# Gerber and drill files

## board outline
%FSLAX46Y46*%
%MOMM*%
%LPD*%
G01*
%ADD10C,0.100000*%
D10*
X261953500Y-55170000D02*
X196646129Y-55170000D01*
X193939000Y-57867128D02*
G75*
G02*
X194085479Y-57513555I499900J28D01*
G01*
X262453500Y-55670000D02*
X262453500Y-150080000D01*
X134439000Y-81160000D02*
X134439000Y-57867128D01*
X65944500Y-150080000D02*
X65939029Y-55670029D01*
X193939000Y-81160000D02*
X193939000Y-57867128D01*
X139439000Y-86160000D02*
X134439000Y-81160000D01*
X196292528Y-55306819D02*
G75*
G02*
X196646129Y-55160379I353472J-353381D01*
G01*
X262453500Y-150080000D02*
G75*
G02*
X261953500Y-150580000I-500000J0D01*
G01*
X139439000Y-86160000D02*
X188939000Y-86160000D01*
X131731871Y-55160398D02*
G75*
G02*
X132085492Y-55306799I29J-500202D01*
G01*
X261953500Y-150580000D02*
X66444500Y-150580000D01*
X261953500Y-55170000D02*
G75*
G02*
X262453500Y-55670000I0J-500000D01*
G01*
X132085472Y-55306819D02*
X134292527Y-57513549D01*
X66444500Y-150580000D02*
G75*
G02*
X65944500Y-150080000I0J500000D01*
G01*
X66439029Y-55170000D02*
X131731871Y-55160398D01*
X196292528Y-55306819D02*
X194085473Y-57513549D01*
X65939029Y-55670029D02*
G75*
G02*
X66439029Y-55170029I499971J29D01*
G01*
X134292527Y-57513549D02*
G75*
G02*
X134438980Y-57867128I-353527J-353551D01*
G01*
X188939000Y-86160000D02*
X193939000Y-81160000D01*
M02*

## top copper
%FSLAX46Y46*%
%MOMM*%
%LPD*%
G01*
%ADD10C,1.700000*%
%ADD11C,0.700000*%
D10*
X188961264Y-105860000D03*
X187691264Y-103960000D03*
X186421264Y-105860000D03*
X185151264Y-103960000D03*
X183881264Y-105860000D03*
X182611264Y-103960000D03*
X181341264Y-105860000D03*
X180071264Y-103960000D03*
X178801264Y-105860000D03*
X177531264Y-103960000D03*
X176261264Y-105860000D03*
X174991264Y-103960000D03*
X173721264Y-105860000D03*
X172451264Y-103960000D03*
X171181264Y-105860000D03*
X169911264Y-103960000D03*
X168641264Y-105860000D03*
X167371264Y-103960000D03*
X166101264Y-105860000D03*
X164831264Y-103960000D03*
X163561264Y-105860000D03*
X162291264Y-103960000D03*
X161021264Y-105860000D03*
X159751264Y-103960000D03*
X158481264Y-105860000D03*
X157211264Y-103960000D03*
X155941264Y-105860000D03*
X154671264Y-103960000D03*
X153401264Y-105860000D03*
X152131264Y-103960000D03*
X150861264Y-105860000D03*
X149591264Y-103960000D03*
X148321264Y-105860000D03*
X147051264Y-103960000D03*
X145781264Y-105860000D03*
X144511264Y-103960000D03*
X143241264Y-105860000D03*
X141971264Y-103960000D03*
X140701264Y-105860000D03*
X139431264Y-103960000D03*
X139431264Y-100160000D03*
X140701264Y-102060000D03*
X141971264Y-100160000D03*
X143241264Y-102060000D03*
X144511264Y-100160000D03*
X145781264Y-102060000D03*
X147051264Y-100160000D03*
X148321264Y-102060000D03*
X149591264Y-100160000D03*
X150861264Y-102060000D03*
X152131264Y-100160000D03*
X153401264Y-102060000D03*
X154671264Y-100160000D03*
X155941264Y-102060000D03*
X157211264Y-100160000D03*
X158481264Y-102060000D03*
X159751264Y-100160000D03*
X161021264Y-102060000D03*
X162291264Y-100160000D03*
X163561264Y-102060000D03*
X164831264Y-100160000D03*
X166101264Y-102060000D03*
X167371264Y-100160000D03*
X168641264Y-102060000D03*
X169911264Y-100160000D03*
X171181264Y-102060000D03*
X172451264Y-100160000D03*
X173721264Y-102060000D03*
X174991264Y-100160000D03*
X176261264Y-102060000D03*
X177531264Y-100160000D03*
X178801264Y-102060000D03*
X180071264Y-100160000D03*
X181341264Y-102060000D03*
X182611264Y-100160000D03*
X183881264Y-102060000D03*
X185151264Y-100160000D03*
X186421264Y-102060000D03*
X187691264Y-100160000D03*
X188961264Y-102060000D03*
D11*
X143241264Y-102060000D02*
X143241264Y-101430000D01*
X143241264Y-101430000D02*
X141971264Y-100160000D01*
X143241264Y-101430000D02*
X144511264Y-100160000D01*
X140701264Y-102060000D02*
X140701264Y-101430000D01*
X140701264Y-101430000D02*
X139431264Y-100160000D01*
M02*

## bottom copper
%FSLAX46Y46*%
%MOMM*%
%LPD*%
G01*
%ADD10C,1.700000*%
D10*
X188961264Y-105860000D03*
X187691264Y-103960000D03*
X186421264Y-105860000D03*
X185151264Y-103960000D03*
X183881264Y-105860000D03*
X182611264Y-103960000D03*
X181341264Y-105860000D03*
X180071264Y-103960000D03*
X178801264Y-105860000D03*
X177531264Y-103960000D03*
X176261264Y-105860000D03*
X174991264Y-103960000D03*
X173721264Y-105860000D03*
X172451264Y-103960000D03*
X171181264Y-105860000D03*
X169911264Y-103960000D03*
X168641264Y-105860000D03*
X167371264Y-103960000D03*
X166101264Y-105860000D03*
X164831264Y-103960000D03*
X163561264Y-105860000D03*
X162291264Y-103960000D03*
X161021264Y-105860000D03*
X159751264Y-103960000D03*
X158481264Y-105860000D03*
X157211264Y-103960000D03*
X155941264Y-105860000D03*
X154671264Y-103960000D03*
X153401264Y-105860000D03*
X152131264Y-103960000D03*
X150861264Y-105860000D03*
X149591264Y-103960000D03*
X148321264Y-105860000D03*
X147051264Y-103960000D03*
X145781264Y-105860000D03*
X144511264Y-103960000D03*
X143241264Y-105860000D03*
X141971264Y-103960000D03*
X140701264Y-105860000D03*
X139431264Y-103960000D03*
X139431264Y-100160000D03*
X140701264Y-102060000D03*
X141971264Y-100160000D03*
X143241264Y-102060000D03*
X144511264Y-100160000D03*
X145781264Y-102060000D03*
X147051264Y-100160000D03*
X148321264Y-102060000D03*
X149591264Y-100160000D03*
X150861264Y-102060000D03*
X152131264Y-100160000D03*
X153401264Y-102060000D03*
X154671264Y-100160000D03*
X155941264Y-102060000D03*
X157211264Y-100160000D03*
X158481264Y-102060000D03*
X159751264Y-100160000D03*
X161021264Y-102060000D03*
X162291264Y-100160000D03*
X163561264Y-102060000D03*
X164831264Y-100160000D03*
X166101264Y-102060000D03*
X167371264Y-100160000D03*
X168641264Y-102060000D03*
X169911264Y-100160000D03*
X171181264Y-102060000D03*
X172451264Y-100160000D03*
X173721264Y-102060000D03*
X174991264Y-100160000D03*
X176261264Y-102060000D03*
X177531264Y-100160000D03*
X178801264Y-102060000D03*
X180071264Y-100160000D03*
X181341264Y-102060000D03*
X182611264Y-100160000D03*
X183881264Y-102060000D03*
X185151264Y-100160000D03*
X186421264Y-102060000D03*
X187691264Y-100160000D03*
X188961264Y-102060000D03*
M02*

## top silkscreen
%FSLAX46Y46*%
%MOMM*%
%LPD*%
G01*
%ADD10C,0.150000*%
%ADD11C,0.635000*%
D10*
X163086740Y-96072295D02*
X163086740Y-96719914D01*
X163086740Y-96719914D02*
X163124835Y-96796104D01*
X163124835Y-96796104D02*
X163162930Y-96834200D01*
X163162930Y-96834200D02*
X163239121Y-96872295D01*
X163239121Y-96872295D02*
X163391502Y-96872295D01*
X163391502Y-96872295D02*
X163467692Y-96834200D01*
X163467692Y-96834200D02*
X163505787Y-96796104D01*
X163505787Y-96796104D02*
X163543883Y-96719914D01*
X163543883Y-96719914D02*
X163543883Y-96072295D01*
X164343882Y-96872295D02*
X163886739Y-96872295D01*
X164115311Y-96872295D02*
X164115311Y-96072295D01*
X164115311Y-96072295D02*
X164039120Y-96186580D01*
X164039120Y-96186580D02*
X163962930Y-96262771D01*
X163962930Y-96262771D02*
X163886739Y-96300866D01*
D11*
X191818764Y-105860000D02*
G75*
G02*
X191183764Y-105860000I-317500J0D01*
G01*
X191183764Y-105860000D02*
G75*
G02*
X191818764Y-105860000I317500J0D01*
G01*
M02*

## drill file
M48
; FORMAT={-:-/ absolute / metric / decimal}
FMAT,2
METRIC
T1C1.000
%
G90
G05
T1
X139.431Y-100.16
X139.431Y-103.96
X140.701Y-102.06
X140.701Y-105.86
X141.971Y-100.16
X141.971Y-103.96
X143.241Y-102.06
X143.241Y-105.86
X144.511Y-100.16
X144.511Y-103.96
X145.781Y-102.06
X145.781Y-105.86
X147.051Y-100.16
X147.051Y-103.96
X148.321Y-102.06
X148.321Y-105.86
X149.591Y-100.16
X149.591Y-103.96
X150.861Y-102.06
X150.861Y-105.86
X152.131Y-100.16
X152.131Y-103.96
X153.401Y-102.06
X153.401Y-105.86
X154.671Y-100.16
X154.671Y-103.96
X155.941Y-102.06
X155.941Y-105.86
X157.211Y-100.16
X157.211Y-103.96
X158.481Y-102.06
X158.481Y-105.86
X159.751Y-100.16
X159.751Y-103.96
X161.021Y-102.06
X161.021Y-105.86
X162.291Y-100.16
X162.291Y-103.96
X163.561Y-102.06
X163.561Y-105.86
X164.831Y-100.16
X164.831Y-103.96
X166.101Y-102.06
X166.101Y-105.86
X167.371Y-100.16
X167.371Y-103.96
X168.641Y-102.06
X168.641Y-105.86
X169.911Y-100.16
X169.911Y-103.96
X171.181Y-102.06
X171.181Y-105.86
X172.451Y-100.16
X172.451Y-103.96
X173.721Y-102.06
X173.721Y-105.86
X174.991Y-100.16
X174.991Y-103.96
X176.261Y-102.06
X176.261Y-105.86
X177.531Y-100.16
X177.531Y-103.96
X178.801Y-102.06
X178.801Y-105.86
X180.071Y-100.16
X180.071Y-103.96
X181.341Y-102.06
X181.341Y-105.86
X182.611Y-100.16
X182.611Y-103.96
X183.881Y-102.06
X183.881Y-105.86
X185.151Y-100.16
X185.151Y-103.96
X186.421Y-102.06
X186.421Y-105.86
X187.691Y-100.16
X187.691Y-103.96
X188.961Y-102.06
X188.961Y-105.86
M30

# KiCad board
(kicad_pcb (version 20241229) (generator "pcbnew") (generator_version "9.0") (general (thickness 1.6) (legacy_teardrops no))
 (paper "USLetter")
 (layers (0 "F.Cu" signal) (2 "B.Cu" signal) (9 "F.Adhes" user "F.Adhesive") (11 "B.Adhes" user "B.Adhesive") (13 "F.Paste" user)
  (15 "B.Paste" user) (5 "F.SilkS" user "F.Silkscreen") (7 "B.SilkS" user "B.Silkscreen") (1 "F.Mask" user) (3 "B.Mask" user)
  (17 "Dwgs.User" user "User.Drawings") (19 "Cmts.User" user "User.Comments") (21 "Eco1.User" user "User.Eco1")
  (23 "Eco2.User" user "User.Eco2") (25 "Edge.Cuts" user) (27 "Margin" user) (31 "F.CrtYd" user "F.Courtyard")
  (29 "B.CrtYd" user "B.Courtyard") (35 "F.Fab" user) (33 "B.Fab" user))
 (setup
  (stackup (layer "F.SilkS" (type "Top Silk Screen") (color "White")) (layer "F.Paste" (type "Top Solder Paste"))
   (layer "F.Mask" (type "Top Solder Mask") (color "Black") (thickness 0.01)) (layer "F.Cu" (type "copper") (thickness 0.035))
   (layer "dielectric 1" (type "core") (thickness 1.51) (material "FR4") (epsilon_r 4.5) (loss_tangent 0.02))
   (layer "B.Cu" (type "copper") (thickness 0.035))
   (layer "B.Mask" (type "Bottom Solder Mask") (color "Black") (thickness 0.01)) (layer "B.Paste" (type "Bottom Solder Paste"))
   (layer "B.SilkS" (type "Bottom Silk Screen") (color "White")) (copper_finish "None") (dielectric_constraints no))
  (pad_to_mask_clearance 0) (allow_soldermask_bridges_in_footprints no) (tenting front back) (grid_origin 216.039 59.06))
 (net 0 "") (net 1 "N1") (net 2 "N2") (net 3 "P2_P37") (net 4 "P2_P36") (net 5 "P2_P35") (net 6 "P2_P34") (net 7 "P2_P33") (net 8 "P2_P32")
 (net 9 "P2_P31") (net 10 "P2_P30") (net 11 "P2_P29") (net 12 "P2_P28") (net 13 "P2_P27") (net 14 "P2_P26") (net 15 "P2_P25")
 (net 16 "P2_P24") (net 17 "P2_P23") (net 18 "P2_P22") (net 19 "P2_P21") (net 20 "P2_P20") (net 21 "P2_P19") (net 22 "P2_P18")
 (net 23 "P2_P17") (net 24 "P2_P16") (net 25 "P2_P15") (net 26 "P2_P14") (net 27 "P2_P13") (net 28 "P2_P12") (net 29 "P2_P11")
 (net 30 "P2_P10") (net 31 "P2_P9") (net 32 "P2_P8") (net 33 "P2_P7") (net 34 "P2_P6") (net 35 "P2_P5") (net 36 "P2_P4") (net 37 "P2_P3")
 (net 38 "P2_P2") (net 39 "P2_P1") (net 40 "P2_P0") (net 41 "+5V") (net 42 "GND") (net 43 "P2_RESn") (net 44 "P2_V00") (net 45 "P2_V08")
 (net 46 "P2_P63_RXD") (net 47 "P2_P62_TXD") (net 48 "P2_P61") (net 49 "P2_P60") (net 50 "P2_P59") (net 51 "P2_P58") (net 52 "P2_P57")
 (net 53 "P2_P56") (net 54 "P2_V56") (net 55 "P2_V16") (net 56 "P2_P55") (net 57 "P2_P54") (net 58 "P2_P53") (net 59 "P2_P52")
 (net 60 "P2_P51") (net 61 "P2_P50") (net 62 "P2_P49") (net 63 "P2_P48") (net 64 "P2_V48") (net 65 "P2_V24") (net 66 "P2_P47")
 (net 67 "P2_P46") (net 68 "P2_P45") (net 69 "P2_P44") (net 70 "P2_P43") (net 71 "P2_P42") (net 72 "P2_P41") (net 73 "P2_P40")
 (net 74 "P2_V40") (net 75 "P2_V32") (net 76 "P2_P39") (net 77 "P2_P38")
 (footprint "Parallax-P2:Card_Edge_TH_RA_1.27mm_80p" (layer "F.Cu") (at 164.196264 103.01)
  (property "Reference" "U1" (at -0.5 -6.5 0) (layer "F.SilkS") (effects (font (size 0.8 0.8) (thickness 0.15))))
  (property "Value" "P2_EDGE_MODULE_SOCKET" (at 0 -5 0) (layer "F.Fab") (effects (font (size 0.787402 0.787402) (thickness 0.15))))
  (fp_circle (center 27.305 2.85) (end 27.94 2.85) (stroke (width 0) (type solid)) (fill yes) (layer "F.SilkS"))
  (pad "1" thru_hole circle (at 24.765 2.85) (size 1.7 1.7) (drill 1) (layers "*.Cu" "*.Mask") (remove_unused_layers no) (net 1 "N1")
   (solder_mask_margin 0.102))
  (pad "2" thru_hole circle (at 23.495 0.95) (size 1.7 1.7) (drill 1) (layers "*.Cu" "*.Mask") (remove_unused_layers no) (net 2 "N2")
   (solder_mask_margin 0.102))
  (pad "3" thru_hole circle (at 22.225 2.85) (size 1.7 1.7) (drill 1) (layers "*.Cu" "*.Mask") (remove_unused_layers no) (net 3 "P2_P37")
   (solder_mask_margin 0.102))
  (pad "4" thru_hole circle (at 20.955 0.95) (size 1.7 1.7) (drill 1) (layers "*.Cu" "*.Mask") (remove_unused_layers no) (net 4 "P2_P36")
   (solder_mask_margin 0.102))
  (pad "5" thru_hole circle (at 19.685 2.85) (size 1.7 1.7) (drill 1) (layers "*.Cu" "*.Mask") (remove_unused_layers no) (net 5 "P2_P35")
   (solder_mask_margin 0.102))
  (pad "6" thru_hole circle (at 18.415 0.95) (size 1.7 1.7) (drill 1) (layers "*.Cu" "*.Mask") (remove_unused_layers no) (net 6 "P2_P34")
   (solder_mask_margin 0.102))
  (pad "7" thru_hole circle (at 17.145 2.85) (size 1.7 1.7) (drill 1) (layers "*.Cu" "*.Mask") (remove_unused_layers no) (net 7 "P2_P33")
   (solder_mask_margin 0.102))
  (pad "8" thru_hole circle (at 15.875 0.95) (size 1.7 1.7) (drill 1) (layers "*.Cu" "*.Mask") (remove_unused_layers no) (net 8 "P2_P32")
   (solder_mask_margin 0.102))
  (pad "9" thru_hole circle (at 14.605 2.85) (size 1.7 1.7) (drill 1) (layers "*.Cu" "*.Mask") (remove_unused_layers no) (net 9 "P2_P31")
   (solder_mask_margin 0.102))
  (pad "10" thru_hole circle (at 13.335 0.95) (size 1.7 1.7) (drill 1) (layers "*.Cu" "*.Mask") (remove_unused_layers no) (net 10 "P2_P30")
   (solder_mask_margin 0.102))
  (pad "11" thru_hole circle (at 12.065 2.85) (size 1.7 1.7) (drill 1) (layers "*.Cu" "*.Mask") (remove_unused_layers no) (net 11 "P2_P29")
   (solder_mask_margin 0.102))
  (pad "12" thru_hole circle (at 10.795 0.95) (size 1.7 1.7) (drill 1) (layers "*.Cu" "*.Mask") (remove_unused_layers no) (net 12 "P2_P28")
   (solder_mask_margin 0.102))
  (pad "13" thru_hole circle (at 9.525 2.85) (size 1.7 1.7) (drill 1) (layers "*.Cu" "*.Mask") (remove_unused_layers no) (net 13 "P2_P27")
   (solder_mask_margin 0.102))
  (pad "14" thru_hole circle (at 8.255 0.95) (size 1.7 1.7) (drill 1) (layers "*.Cu" "*.Mask") (remove_unused_layers no) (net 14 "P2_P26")
   (solder_mask_margin 0.102))
  (pad "15" thru_hole circle (at 6.985 2.85) (size 1.7 1.7) (drill 1) (layers "*.Cu" "*.Mask") (remove_unused_layers no) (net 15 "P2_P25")
   (solder_mask_margin 0.102))
  (pad "16" thru_hole circle (at 5.715 0.95) (size 1.7 1.7) (drill 1) (layers "*.Cu" "*.Mask") (remove_unused_layers no) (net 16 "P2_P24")
   (solder_mask_margin 0.102))
  (pad "17" thru_hole circle (at 4.445 2.85) (size 1.7 1.7) (drill 1) (layers "*.Cu" "*.Mask") (remove_unused_layers no) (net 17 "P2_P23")
   (solder_mask_margin 0.102))
  (pad "18" thru_hole circle (at 3.175 0.95) (size 1.7 1.7) (drill 1) (layers "*.Cu" "*.Mask") (remove_unused_layers no) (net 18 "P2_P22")
   (solder_mask_margin 0.102))
  (pad "19" thru_hole circle (at 1.905 2.85) (size 1.7 1.7) (drill 1) (layers "*.Cu" "*.Mask") (remove_unused_layers no) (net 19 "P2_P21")
   (solder_mask_margin 0.102))
  (pad "20" thru_hole circle (at 0.635 0.95) (size 1.7 1.7) (drill 1) (layers "*.Cu" "*.Mask") (remove_unused_layers no) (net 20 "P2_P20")
   (solder_mask_margin 0.102))
  (pad "21" thru_hole circle (at -0.635 2.85) (size 1.7 1.7) (drill 1) (layers "*.Cu" "*.Mask") (remove_unused_layers no) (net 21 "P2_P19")
   (solder_mask_margin 0.102))
  (pad "22" thru_hole circle (at -1.905 0.95) (size 1.7 1.7) (drill 1) (layers "*.Cu" "*.Mask") (remove_unused_layers no) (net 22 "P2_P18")
   (solder_mask_margin 0.102))
  (pad "23" thru_hole circle (at -3.175 2.85) (size 1.7 1.7) (drill 1) (layers "*.Cu" "*.Mask") (remove_unused_layers no) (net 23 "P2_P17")
   (solder_mask_margin 0.102))
  (pad "24" thru_hole circle (at -4.445 0.95) (size 1.7 1.7) (drill 1) (layers "*.Cu" "*.Mask") (remove_unused_layers no) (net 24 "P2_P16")
   (solder_mask_margin 0.102))
  (pad "25" thru_hole circle (at -5.715 2.85) (size 1.7 1.7) (drill 1) (layers "*.Cu" "*.Mask") (remove_unused_layers no) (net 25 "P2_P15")
   (solder_mask_margin 0.102))
  (pad "26" thru_hole circle (at -6.985 0.95) (size 1.7 1.7) (drill 1) (layers "*.Cu" "*.Mask") (remove_unused_layers no) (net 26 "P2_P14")
   (solder_mask_margin 0.102))
  (pad "27" thru_hole circle (at -8.255 2.85) (size 1.7 1.7) (drill 1) (layers "*.Cu" "*.Mask") (remove_unused_layers no) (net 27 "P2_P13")
   (solder_mask_margin 0.102))
  (pad "28" thru_hole circle (at -9.525 0.95) (size 1.7 1.7) (drill 1) (layers "*.Cu" "*.Mask") (remove_unused_layers no) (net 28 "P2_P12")
   (solder_mask_margin 0.102))
  (pad "29" thru_hole circle (at -10.795 2.85) (size 1.7 1.7) (drill 1) (layers "*.Cu" "*.Mask") (remove_unused_layers no) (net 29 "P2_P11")
   (solder_mask_margin 0.102))
  (pad "30" thru_hole circle (at -12.065 0.95) (size 1.7 1.7) (drill 1) (layers "*.Cu" "*.Mask") (remove_unused_layers no) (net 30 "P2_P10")
   (solder_mask_margin 0.102))
  (pad "31" thru_hole circle (at -13.335 2.85) (size 1.7 1.7) (drill 1) (layers "*.Cu" "*.Mask") (remove_unused_layers no) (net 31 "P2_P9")
   (solder_mask_margin 0.102))
  (pad "32" thru_hole circle (at -14.605 0.95) (size 1.7 1.7) (drill 1) (layers "*.Cu" "*.Mask") (remove_unused_layers no) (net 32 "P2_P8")
   (solder_mask_margin 0.102))
  (pad "33" thru_hole circle (at -15.875 2.85) (size 1.7 1.7) (drill 1) (layers "*.Cu" "*.Mask") (remove_unused_layers no) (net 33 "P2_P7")
   (solder_mask_margin 0.102))
  (pad "34" thru_hole circle (at -17.145 0.95) (size 1.7 1.7) (drill 1) (layers "*.Cu" "*.Mask") (remove_unused_layers no) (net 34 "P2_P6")
   (solder_mask_margin 0.102))
  (pad "35" thru_hole circle (at -18.415 2.85) (size 1.7 1.7) (drill 1) (layers "*.Cu" "*.Mask") (remove_unused_layers no) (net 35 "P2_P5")
   (solder_mask_margin 0.102))
  (pad "36" thru_hole circle (at -19.685 0.95) (size 1.7 1.7) (drill 1) (layers "*.Cu" "*.Mask") (remove_unused_layers no) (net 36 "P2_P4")
   (solder_mask_margin 0.102))
  (pad "37" thru_hole circle (at -20.955 2.85) (size 1.7 1.7) (drill 1) (layers "*.Cu" "*.Mask") (remove_unused_layers no) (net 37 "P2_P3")
   (solder_mask_margin 0.102))
  (pad "38" thru_hole circle (at -22.225 0.95) (size 1.7 1.7) (drill 1) (layers "*.Cu" "*.Mask") (remove_unused_layers no) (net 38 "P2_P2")
   (solder_mask_margin 0.102))
  (pad "39" thru_hole circle (at -23.495 2.85) (size 1.7 1.7) (drill 1) (layers "*.Cu" "*.Mask") (remove_unused_layers no) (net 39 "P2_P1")
   (solder_mask_margin 0.102))
  (pad "40" thru_hole circle (at -24.765 0.95) (size 1.7 1.7) (drill 1) (layers "*.Cu" "*.Mask") (remove_unused_layers no) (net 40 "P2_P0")
   (solder_mask_margin 0.102))
  (pad "41" thru_hole circle (at -24.765 -2.85) (size 1.7 1.7) (drill 1) (layers "*.Cu" "*.Mask") (remove_unused_layers no) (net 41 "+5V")
   (solder_mask_margin 0.102))
  (pad "42" thru_hole circle (at -23.495 -0.95) (size 1.7 1.7) (drill 1) (layers "*.Cu" "*.Mask") (remove_unused_layers no) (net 41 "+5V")
   (solder_mask_margin 0.102))
  (pad "43" thru_hole circle (at -22.225 -2.85) (size 1.7 1.7) (drill 1) (layers "*.Cu" "*.Mask") (remove_unused_layers no) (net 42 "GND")
   (solder_mask_margin 0.102))
  (pad "44" thru_hole circle (at -20.955 -0.95) (size 1.7 1.7) (drill 1) (layers "*.Cu" "*.Mask") (remove_unused_layers no) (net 42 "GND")
   (solder_mask_margin 0.102))
  (pad "45" thru_hole circle (at -19.685 -2.85) (size 1.7 1.7) (drill 1) (layers "*.Cu" "*.Mask") (remove_unused_layers no) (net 42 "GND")
   (solder_mask_margin 0.102))
  (pad "46" thru_hole circle (at -18.415 -0.95) (size 1.7 1.7) (drill 1) (layers "*.Cu" "*.Mask") (remove_unused_layers no)
   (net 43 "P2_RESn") (solder_mask_margin 0.102))
  (pad "47" thru_hole circle (at -17.145 -2.85) (size 1.7 1.7) (drill 1) (layers "*.Cu" "*.Mask") (remove_unused_layers no)
   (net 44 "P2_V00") (solder_mask_margin 0.102))
  (pad "48" thru_hole circle (at -15.875 -0.95) (size 1.7 1.7) (drill 1) (layers "*.Cu" "*.Mask") (remove_unused_layers no)
   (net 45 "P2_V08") (solder_mask_margin 0.102))
  (pad "49" thru_hole circle (at -14.605 -2.85) (size 1.7 1.7) (drill 1) (layers "*.Cu" "*.Mask") (remove_unused_layers no)
   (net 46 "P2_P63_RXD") (solder_mask_margin 0.102))
  (pad "50" thru_hole circle (at -13.335 -0.95) (size 1.7 1.7) (drill 1) (layers "*.Cu" "*.Mask") (remove_unused_layers no)
   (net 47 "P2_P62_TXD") (solder_mask_margin 0.102))
  (pad "51" thru_hole circle (at -12.065 -2.85) (size 1.7 1.7) (drill 1) (layers "*.Cu" "*.Mask") (remove_unused_layers no)
   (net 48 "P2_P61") (solder_mask_margin 0.102))
  (pad "52" thru_hole circle (at -10.795 -0.95) (size 1.7 1.7) (drill 1) (layers "*.Cu" "*.Mask") (remove_unused_layers no)
   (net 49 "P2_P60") (solder_mask_margin 0.102))
  (pad "53" thru_hole circle (at -9.525 -2.85) (size 1.7 1.7) (drill 1) (layers "*.Cu" "*.Mask") (remove_unused_layers no) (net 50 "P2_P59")
   (solder_mask_margin 0.102))
  (pad "54" thru_hole circle (at -8.255 -0.95) (size 1.7 1.7) (drill 1) (layers "*.Cu" "*.Mask") (remove_unused_layers no) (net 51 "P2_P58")
   (solder_mask_margin 0.102))
  (pad "55" thru_hole circle (at -6.985 -2.85) (size 1.7 1.7) (drill 1) (layers "*.Cu" "*.Mask") (remove_unused_layers no) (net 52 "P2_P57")
   (solder_mask_margin 0.102))
  (pad "56" thru_hole circle (at -5.715 -0.95) (size 1.7 1.7) (drill 1) (layers "*.Cu" "*.Mask") (remove_unused_layers no) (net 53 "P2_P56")
   (solder_mask_margin 0.102))
  (pad "57" thru_hole circle (at -4.445 -2.85) (size 1.7 1.7) (drill 1) (layers "*.Cu" "*.Mask") (remove_unused_layers no) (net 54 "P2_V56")
   (solder_mask_margin 0.102))
  (pad "58" thru_hole circle (at -3.175 -0.95) (size 1.7 1.7) (drill 1) (layers "*.Cu" "*.Mask") (remove_unused_layers no) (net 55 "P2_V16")
   (solder_mask_margin 0.102))
  (pad "59" thru_hole circle (at -1.905 -2.85) (size 1.7 1.7) (drill 1) (layers "*.Cu" "*.Mask") (remove_unused_layers no) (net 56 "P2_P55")
   (solder_mask_margin 0.102))
  (pad "60" thru_hole circle (at -0.635 -0.95) (size 1.7 1.7) (drill 1) (layers "*.Cu" "*.Mask") (remove_unused_layers no) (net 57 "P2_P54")
   (solder_mask_margin 0.102))
  (pad "61" thru_hole circle (at 0.635 -2.85) (size 1.7 1.7) (drill 1) (layers "*.Cu" "*.Mask") (remove_unused_layers no) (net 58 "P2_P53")
   (solder_mask_margin 0.102))
  (pad "62" thru_hole circle (at 1.905 -0.95) (size 1.7 1.7) (drill 1) (layers "*.Cu" "*.Mask") (remove_unused_layers no) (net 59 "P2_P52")
   (solder_mask_margin 0.102))
  (pad "63" thru_hole circle (at 3.175 -2.85) (size 1.7 1.7) (drill 1) (layers "*.Cu" "*.Mask") (remove_unused_layers no) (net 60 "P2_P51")
   (solder_mask_margin 0.102))
  (pad "64" thru_hole circle (at 4.445 -0.95) (size 1.7 1.7) (drill 1) (layers "*.Cu" "*.Mask") (remove_unused_layers no) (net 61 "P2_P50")
   (solder_mask_margin 0.102))
  (pad "65" thru_hole circle (at 5.715 -2.85) (size 1.7 1.7) (drill 1) (layers "*.Cu" "*.Mask") (remove_unused_layers no) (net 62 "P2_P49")
   (solder_mask_margin 0.102))
  (pad "66" thru_hole circle (at 6.985 -0.95) (size 1.7 1.7) (drill 1) (layers "*.Cu" "*.Mask") (remove_unused_layers no) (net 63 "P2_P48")
   (solder_mask_margin 0.102))
  (pad "67" thru_hole circle (at 8.255 -2.85) (size 1.7 1.7) (drill 1) (layers "*.Cu" "*.Mask") (remove_unused_layers no) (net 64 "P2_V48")
   (solder_mask_margin 0.102))
  (pad "68" thru_hole circle (at 9.525 -0.95) (size 1.7 1.7) (drill 1) (layers "*.Cu" "*.Mask") (remove_unused_layers no) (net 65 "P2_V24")
   (solder_mask_margin 0.102))
  (pad "69" thru_hole circle (at 10.795 -2.85) (size 1.7 1.7) (drill 1) (layers "*.Cu" "*.Mask") (remove_unused_layers no) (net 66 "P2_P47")
   (solder_mask_margin 0.102))
  (pad "70" thru_hole circle (at 12.065 -0.95) (size 1.7 1.7) (drill 1) (layers "*.Cu" "*.Mask") (remove_unused_layers no) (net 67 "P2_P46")
   (solder_mask_margin 0.102))
  (pad "71" thru_hole circle (at 13.335 -2.85) (size 1.7 1.7) (drill 1) (layers "*.Cu" "*.Mask") (remove_unused_layers no) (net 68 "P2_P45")
   (solder_mask_margin 0.102))
  (pad "72" thru_hole circle (at 14.605 -0.95) (size 1.7 1.7) (drill 1) (layers "*.Cu" "*.Mask") (remove_unused_layers no) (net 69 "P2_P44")
   (solder_mask_margin 0.102))
  (pad "73" thru_hole circle (at 15.875 -2.85) (size 1.7 1.7) (drill 1) (layers "*.Cu" "*.Mask") (remove_unused_layers no) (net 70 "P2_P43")
   (solder_mask_margin 0.102))
  (pad "74" thru_hole circle (at 17.145 -0.95) (size 1.7 1.7) (drill 1) (layers "*.Cu" "*.Mask") (remove_unused_layers no) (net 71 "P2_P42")
   (solder_mask_margin 0.102))
  (pad "75" thru_hole circle (at 18.415 -2.85) (size 1.7 1.7) (drill 1) (layers "*.Cu" "*.Mask") (remove_unused_layers no) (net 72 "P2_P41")
   (solder_mask_margin 0.102))
  (pad "76" thru_hole circle (at 19.685 -0.95) (size 1.7 1.7) (drill 1) (layers "*.Cu" "*.Mask") (remove_unused_layers no) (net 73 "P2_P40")
   (solder_mask_margin 0.102))
  (pad "77" thru_hole circle (at 20.955 -2.85) (size 1.7 1.7) (drill 1) (layers "*.Cu" "*.Mask") (remove_unused_layers no) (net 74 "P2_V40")
   (solder_mask_margin 0.102))
  (pad "78" thru_hole circle (at 22.225 -0.95) (size 1.7 1.7) (drill 1) (layers "*.Cu" "*.Mask") (remove_unused_layers no) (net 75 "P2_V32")
   (solder_mask_margin 0.102))
  (pad "79" thru_hole circle (at 23.495 -2.85) (size 1.7 1.7) (drill 1) (layers "*.Cu" "*.Mask") (remove_unused_layers no) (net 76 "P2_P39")
   (solder_mask_margin 0.102))
  (pad "80" thru_hole circle (at 24.765 -0.95) (size 1.7 1.7) (drill 1) (layers "*.Cu" "*.Mask") (remove_unused_layers no) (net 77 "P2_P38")
   (solder_mask_margin 0.102)))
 (gr_line (start 261.9535 55.17) (end 196.646129 55.17) (stroke (width 0.1) (type solid)) (layer "Edge.Cuts"))
 (gr_arc (start 193.939 57.867128) (mid 193.977058 57.675763) (end 194.085473 57.513549) (stroke (width 0.1) (type default))
  (layer "Edge.Cuts"))
 (gr_line (start 262.4535 55.67) (end 262.4535 150.08) (stroke (width 0.1) (type solid)) (layer "Edge.Cuts"))
 (gr_line (start 134.439 81.16) (end 134.439 57.867128) (stroke (width 0.1) (type solid)) (layer "Edge.Cuts"))
 (gr_line (start 65.9445 150.08) (end 65.939029 55.670029) (stroke (width 0.1) (type solid)) (layer "Edge.Cuts"))
 (gr_line (start 193.939 81.16) (end 193.939 57.867128) (stroke (width 0.1) (type solid)) (layer "Edge.Cuts"))
 (gr_line (start 139.439 86.16) (end 134.439 81.16) (stroke (width 0.1) (type default)) (layer "Edge.Cuts"))
 (gr_arc (start 196.292528 55.306819) (mid 196.454762 55.198423) (end 196.646129 55.160398) (stroke (width 0.1) (type default))
  (layer "Edge.Cuts"))
 (gr_arc (start 262.4535 150.08) (mid 262.307053 150.433553) (end 261.9535 150.58) (stroke (width 0.1) (type solid)) (layer "Edge.Cuts"))
 (gr_line (start 139.439 86.16) (end 188.939 86.16) (stroke (width 0.1) (type default)) (layer "Edge.Cuts"))
 (gr_arc (start 131.731871 55.160398) (mid 131.923226 55.198452) (end 132.085472 55.306819) (stroke (width 0.1) (type default))
  (layer "Edge.Cuts"))
 (gr_line (start 261.9535 150.58) (end 66.4445 150.58) (stroke (width 0.1) (type solid)) (layer "Edge.Cuts"))
 (gr_arc (start 261.9535 55.17) (mid 262.307053 55.316447) (end 262.4535 55.67) (stroke (width 0.1) (type solid)) (layer "Edge.Cuts"))
 (gr_line (start 132.085472 55.306819) (end 134.292527 57.513549) (stroke (width 0.1) (type default)) (layer "Edge.Cuts"))
 (gr_arc (start 66.4445 150.58) (mid 66.090947 150.433553) (end 65.9445 150.08) (stroke (width 0.1) (type solid)) (layer "Edge.Cuts"))
 (gr_line (start 66.439029 55.17) (end 131.731871 55.160398) (stroke (width 0.1) (type default)) (layer "Edge.Cuts"))
 (gr_line (start 196.292528 55.306819) (end 194.085473 57.513549) (stroke (width 0.1) (type default)) (layer "Edge.Cuts"))
 (gr_arc (start 65.939029 55.670029) (mid 66.085467 55.316467) (end 66.439029 55.17) (stroke (width 0.1) (type solid)) (layer "Edge.Cuts"))
 (gr_arc (start 134.292527 57.513549) (mid 134.400932 57.67577) (end 134.439 57.867128) (stroke (width 0.1) (type default))
  (layer "Edge.Cuts"))
 (gr_line (start 188.939 86.16) (end 193.939 81.16) (stroke (width 0.1) (type default)) (layer "Edge.Cuts"))
 (segment (start 143.241264 102.06) (end 143.241264 101.43) (width 0.7) (layer "F.Cu") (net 42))
 (segment (start 143.241264 101.43) (end 141.971264 100.16) (width 0.7) (layer "F.Cu") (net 42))
 (segment (start 143.241264 101.43) (end 144.511264 100.16) (width 0.7) (layer "F.Cu") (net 42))
 (segment (start 140.701264 102.06) (end 140.701264 101.43) (width 0.7) (layer "F.Cu") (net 41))
 (segment (start 140.701264 101.43) (end 139.431264 100.16) (width 0.7) (layer "F.Cu") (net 41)))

